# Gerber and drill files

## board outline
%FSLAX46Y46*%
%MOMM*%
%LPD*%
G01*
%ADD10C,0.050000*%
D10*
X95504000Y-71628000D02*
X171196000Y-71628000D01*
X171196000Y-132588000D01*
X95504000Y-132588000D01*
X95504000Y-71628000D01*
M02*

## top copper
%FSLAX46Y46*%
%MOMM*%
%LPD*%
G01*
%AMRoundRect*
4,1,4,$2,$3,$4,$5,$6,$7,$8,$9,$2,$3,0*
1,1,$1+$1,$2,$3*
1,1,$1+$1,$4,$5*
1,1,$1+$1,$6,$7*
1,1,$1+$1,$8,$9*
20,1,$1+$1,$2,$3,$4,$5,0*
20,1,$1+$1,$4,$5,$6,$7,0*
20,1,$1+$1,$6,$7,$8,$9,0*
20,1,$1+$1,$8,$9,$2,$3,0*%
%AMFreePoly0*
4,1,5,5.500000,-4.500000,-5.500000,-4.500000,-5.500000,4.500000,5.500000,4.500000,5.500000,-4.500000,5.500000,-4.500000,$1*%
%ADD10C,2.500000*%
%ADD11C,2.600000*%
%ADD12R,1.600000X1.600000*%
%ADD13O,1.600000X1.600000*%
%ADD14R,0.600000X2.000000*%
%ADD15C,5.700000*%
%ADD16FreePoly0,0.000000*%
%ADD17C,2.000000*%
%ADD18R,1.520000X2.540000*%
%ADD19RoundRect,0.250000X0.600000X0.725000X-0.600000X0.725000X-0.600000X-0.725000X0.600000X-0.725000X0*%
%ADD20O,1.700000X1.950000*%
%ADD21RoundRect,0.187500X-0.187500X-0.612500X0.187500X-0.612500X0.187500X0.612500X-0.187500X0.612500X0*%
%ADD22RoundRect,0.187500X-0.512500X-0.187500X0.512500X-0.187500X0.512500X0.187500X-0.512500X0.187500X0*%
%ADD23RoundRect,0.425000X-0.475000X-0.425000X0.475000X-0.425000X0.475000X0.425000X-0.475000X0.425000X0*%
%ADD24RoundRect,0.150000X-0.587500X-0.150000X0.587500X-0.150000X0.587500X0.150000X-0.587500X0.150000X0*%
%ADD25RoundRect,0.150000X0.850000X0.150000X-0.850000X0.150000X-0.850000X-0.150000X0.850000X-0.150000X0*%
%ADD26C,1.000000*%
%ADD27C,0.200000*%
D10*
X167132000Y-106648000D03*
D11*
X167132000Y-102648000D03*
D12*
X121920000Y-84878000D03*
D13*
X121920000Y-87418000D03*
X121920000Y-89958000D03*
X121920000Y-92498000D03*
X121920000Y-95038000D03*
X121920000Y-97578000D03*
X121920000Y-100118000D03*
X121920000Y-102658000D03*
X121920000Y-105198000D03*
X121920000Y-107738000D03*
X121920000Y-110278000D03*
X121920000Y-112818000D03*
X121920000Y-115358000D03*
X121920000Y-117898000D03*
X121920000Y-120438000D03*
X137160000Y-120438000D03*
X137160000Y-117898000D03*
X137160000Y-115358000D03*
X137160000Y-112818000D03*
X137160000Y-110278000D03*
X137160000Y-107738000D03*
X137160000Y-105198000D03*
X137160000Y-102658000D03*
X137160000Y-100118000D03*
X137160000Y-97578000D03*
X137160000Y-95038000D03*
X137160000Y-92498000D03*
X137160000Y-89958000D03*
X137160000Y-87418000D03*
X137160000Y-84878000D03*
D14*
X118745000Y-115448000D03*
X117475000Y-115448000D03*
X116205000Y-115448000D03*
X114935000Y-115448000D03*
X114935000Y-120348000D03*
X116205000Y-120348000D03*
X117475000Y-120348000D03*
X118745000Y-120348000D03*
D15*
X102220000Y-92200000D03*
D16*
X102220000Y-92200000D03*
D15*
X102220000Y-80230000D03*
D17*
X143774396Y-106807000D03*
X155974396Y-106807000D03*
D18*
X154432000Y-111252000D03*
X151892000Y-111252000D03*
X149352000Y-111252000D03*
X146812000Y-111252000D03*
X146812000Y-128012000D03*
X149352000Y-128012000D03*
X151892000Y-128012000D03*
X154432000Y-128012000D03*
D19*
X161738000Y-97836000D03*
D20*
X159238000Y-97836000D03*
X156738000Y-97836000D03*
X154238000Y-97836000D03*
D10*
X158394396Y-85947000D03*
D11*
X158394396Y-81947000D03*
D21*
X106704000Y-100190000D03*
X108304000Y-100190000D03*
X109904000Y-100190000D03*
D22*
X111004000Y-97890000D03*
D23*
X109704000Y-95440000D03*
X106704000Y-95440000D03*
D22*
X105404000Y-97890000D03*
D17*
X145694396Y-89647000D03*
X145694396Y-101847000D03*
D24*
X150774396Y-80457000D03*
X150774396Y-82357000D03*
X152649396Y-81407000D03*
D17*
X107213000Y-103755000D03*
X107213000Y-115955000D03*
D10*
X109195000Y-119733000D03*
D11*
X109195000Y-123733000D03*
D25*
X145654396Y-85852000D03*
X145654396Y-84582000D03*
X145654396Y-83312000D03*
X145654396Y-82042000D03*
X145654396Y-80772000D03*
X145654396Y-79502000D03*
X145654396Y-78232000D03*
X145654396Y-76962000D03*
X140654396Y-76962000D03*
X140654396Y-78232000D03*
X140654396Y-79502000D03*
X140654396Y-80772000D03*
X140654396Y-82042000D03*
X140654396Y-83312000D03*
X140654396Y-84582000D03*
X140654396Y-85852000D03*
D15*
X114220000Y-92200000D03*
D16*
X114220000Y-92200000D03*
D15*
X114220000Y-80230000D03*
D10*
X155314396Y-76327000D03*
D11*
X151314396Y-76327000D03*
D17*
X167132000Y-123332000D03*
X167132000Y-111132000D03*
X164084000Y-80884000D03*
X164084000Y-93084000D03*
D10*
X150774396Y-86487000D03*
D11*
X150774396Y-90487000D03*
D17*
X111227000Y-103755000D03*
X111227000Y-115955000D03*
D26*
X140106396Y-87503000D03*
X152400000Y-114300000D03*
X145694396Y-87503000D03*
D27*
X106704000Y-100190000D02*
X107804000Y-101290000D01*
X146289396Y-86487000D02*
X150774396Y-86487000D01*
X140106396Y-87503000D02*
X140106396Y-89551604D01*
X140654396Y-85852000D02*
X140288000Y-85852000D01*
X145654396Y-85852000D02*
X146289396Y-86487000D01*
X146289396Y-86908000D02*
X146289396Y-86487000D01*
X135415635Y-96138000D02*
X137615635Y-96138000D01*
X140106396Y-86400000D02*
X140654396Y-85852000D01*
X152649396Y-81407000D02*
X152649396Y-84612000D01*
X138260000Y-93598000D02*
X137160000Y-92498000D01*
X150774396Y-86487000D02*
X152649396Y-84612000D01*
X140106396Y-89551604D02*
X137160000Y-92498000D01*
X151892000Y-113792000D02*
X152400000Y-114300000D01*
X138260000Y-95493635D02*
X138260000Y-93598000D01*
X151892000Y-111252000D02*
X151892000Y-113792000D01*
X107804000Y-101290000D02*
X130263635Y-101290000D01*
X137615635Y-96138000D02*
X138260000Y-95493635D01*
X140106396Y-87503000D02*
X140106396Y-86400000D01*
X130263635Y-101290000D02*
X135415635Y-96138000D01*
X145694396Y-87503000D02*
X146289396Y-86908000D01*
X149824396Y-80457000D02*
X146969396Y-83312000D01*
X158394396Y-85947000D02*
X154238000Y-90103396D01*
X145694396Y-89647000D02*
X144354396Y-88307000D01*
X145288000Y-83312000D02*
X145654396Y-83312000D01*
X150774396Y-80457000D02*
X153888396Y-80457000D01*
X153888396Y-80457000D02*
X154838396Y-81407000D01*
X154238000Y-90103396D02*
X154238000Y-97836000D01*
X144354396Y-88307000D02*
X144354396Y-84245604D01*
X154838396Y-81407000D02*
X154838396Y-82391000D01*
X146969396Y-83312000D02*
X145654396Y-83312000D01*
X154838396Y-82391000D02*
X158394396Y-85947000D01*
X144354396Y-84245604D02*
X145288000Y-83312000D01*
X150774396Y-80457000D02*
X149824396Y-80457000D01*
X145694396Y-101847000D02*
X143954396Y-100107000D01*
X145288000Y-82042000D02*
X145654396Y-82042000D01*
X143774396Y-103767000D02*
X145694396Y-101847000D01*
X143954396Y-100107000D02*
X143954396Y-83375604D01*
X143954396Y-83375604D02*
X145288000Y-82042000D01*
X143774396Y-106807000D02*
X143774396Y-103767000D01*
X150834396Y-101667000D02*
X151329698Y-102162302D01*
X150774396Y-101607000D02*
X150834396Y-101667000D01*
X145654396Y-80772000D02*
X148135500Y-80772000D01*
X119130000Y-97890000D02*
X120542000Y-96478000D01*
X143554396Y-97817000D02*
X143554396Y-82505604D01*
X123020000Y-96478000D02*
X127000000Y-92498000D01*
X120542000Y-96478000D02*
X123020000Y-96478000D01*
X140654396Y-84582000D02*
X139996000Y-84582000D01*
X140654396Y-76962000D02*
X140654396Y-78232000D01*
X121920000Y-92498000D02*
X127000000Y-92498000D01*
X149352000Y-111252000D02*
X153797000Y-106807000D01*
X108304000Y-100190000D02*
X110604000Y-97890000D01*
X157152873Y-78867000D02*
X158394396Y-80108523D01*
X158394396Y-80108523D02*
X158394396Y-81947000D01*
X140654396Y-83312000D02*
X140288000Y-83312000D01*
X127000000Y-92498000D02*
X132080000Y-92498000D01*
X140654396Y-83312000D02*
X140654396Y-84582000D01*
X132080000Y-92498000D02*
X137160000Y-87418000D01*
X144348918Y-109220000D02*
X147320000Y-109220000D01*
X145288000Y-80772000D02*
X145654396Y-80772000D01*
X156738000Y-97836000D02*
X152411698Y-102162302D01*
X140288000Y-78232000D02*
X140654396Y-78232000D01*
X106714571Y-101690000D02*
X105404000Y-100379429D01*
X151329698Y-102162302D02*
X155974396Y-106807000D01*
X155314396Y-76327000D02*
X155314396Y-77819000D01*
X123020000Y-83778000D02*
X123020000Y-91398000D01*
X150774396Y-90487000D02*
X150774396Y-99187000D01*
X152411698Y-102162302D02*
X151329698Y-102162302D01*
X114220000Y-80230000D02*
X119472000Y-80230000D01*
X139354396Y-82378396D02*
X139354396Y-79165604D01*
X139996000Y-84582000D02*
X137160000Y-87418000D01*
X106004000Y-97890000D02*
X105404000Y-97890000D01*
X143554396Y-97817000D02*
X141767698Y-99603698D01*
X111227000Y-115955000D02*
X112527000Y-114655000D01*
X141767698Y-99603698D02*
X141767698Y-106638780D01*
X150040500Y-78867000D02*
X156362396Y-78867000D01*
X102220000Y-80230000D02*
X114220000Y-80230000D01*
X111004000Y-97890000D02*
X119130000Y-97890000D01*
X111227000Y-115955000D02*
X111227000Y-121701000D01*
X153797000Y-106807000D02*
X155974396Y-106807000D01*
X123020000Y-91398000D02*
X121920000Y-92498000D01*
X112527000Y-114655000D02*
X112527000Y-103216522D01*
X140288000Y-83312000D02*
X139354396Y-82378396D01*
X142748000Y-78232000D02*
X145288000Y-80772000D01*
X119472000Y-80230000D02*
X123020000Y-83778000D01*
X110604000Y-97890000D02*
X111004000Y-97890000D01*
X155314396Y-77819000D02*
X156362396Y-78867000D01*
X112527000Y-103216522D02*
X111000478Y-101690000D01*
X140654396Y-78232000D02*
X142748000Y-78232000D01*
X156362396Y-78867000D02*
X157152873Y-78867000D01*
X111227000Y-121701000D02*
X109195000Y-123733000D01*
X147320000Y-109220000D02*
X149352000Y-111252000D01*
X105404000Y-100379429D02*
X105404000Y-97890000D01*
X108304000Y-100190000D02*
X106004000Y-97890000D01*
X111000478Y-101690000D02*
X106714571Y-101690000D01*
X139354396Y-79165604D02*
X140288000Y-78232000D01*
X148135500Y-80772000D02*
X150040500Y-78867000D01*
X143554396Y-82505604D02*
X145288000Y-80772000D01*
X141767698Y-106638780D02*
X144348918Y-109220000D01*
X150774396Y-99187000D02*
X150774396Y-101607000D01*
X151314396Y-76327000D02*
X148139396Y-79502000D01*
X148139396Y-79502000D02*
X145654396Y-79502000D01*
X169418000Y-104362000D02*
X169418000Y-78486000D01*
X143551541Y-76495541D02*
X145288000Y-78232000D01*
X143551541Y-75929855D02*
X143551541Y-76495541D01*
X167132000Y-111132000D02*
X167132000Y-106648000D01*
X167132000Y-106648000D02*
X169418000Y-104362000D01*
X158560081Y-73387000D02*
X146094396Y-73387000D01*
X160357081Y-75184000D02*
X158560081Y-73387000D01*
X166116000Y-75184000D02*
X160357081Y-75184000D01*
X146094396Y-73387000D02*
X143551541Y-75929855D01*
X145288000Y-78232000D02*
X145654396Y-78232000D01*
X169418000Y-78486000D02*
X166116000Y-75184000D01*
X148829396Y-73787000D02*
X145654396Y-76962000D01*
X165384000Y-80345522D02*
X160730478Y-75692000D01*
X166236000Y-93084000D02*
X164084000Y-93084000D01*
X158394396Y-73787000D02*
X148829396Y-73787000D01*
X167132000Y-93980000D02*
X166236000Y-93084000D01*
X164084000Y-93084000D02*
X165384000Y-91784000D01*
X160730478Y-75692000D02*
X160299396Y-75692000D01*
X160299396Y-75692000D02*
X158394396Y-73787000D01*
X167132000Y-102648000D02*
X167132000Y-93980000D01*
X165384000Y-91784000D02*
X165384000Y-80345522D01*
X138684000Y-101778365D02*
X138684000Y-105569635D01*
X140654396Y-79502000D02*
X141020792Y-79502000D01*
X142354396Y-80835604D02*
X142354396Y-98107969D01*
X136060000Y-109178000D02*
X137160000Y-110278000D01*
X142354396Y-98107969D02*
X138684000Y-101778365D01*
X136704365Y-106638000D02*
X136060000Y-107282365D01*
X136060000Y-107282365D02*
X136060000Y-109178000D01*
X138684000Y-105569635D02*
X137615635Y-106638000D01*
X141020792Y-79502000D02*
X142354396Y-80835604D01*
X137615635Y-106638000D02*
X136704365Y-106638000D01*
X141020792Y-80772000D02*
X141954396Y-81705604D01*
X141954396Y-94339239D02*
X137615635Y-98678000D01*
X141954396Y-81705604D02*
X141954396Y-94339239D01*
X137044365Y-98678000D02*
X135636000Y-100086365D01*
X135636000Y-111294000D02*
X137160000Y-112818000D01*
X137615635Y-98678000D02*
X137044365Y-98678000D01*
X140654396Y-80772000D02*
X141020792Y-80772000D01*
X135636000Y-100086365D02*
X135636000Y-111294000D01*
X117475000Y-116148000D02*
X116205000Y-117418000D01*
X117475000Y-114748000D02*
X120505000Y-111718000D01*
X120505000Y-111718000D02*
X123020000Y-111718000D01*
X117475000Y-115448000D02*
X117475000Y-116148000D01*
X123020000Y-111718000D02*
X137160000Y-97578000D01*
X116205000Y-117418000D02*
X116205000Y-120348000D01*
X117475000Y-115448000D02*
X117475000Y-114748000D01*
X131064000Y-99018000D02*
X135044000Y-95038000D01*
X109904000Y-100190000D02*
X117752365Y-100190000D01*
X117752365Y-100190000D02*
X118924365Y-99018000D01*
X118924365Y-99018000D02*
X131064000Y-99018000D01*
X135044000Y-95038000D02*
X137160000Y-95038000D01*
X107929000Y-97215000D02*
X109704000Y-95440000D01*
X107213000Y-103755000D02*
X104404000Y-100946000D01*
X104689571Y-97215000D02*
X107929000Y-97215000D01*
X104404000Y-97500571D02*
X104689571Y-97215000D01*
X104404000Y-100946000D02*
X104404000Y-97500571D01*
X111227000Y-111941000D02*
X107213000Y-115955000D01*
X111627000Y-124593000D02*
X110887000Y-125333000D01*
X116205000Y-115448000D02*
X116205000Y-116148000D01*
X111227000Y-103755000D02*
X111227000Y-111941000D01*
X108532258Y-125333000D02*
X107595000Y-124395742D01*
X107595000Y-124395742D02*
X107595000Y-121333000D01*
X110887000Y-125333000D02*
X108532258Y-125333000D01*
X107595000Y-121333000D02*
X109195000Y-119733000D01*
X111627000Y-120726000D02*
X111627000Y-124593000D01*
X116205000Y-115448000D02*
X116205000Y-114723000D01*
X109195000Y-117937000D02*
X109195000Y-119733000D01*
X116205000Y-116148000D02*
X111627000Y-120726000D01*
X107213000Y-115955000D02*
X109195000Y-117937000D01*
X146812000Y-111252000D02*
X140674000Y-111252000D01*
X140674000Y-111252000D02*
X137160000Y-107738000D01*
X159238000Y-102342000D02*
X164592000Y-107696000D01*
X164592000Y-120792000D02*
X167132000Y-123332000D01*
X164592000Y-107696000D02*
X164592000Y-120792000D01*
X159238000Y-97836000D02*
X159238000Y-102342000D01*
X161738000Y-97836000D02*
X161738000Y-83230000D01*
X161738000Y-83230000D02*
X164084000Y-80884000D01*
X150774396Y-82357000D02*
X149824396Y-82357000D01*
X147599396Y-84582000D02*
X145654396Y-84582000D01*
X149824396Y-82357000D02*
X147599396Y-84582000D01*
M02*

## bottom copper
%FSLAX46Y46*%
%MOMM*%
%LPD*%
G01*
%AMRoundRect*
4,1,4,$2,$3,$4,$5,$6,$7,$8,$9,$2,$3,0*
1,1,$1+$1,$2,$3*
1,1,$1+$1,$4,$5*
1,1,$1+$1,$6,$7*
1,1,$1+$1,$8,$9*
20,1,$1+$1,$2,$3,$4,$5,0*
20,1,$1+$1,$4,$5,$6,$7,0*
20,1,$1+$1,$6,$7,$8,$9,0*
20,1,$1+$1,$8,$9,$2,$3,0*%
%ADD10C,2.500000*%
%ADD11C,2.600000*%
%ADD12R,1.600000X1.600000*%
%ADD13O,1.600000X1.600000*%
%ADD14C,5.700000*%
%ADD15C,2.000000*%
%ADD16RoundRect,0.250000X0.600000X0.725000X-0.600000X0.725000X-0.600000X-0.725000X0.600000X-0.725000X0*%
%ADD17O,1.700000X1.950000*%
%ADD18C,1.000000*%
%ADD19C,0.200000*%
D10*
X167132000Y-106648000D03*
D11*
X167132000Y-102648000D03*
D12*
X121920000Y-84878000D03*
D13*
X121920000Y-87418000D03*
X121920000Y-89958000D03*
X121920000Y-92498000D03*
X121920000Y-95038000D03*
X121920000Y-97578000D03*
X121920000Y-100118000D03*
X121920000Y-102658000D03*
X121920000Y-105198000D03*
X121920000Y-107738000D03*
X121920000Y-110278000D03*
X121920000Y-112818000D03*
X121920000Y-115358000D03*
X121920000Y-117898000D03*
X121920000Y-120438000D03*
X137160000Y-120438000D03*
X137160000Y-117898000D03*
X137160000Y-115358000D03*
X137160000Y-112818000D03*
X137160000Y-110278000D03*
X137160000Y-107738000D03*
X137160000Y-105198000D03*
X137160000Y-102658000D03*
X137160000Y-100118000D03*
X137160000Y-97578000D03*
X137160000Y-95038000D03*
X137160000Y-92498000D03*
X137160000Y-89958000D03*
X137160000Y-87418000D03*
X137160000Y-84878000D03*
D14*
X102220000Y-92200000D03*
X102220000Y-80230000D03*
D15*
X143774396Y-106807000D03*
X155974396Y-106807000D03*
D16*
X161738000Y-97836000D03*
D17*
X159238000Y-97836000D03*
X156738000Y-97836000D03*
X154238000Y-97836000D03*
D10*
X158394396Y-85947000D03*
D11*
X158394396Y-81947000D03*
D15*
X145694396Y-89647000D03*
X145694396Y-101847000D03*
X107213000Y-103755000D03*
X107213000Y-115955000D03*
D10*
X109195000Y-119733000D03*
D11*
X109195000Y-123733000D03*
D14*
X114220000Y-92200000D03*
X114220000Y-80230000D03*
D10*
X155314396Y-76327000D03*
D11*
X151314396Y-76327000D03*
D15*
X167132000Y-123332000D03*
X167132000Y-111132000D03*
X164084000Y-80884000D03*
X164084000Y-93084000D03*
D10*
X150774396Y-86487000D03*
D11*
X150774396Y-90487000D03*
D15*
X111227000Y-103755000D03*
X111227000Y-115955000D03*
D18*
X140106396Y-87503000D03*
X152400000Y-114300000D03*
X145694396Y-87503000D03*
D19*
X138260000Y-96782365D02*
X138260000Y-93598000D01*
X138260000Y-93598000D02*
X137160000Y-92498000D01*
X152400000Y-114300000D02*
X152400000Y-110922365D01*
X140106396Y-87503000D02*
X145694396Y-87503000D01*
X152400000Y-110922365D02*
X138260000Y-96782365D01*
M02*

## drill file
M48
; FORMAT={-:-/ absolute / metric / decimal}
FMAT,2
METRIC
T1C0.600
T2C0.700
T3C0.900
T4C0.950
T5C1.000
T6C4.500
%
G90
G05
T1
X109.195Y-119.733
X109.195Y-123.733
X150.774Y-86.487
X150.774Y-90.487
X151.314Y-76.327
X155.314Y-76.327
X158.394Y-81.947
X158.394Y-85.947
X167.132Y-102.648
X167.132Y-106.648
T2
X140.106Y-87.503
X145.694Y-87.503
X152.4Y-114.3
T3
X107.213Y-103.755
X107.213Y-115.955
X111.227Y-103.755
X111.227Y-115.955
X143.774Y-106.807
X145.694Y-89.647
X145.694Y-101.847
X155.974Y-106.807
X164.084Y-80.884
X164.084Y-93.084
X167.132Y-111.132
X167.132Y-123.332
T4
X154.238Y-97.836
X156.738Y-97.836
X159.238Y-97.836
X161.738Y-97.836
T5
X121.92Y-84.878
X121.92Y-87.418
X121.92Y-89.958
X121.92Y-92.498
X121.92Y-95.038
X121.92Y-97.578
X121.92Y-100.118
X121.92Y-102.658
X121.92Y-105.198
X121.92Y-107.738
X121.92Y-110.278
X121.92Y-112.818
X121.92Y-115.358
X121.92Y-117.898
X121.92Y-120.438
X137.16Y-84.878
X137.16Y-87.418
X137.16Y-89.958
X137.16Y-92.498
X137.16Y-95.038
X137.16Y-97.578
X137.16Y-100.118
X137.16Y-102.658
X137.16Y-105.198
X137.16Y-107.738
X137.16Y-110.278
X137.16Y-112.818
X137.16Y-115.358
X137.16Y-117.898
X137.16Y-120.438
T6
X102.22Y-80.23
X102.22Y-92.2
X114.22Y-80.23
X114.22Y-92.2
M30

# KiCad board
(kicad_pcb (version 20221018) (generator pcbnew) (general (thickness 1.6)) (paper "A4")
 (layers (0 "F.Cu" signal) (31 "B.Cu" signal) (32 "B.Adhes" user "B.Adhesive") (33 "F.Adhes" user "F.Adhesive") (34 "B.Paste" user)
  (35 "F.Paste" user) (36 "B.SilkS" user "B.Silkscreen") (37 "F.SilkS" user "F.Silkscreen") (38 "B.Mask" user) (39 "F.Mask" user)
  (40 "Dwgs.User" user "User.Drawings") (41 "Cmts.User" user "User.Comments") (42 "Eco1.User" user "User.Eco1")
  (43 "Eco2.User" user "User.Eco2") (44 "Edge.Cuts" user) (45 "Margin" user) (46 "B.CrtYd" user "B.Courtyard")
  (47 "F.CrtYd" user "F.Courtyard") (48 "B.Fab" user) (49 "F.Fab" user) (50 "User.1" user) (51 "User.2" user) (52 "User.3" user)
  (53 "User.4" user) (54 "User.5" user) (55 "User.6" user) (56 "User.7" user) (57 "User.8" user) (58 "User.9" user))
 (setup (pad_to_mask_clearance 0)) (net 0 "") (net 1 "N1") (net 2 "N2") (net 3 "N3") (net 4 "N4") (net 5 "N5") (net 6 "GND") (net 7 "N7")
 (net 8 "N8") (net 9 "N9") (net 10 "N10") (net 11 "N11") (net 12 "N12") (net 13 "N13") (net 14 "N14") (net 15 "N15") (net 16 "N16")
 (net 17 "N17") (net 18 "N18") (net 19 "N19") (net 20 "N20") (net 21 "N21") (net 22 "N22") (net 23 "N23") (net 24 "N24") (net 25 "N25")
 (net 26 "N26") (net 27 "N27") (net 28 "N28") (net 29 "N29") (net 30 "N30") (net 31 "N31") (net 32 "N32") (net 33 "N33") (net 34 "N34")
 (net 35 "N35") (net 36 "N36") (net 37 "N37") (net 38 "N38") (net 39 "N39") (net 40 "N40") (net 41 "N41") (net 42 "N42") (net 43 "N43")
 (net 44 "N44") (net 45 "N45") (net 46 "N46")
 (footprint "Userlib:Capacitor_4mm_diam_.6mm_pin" (layer "F.Cu") (at 167.132 104.648 90)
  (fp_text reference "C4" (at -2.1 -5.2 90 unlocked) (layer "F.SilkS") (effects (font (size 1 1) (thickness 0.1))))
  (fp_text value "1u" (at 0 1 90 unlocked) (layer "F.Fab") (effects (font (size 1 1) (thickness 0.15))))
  (pad "1" thru_hole circle (at -2 0 90) (size 2.5 2.5) (drill 0.6) (layers "*.Cu" "*.Mask") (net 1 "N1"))
  (pad "2" thru_hole circle (at 2 0 90) (size 2.6 2.6) (drill 0.6) (layers "*.Cu" "*.Mask") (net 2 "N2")))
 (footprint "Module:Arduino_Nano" (layer "F.Cu") (at 121.92 84.878)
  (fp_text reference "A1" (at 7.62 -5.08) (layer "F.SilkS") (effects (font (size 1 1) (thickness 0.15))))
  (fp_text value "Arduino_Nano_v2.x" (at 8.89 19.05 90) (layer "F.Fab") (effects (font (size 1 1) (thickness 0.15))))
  (pad "1" thru_hole rect (at 0 0) (size 1.6 1.6) (drill 1) (layers "*.Cu" "*.Mask") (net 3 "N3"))
  (pad "2" thru_hole oval (at 0 2.54) (size 1.6 1.6) (drill 1) (layers "*.Cu" "*.Mask") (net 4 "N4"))
  (pad "3" thru_hole oval (at 0 5.08) (size 1.6 1.6) (drill 1) (layers "*.Cu" "*.Mask") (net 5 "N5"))
  (pad "4" thru_hole oval (at 0 7.62) (size 1.6 1.6) (drill 1) (layers "*.Cu" "*.Mask") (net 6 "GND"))
  (pad "5" thru_hole oval (at 0 10.16) (size 1.6 1.6) (drill 1) (layers "*.Cu" "*.Mask") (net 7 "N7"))
  (pad "6" thru_hole oval (at 0 12.7) (size 1.6 1.6) (drill 1) (layers "*.Cu" "*.Mask") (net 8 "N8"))
  (pad "7" thru_hole oval (at 0 15.24) (size 1.6 1.6) (drill 1) (layers "*.Cu" "*.Mask") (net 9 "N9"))
  (pad "8" thru_hole oval (at 0 17.78) (size 1.6 1.6) (drill 1) (layers "*.Cu" "*.Mask") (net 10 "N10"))
  (pad "9" thru_hole oval (at 0 20.32) (size 1.6 1.6) (drill 1) (layers "*.Cu" "*.Mask") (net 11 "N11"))
  (pad "10" thru_hole oval (at 0 22.86) (size 1.6 1.6) (drill 1) (layers "*.Cu" "*.Mask") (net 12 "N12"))
  (pad "11" thru_hole oval (at 0 25.4) (size 1.6 1.6) (drill 1) (layers "*.Cu" "*.Mask") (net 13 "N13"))
  (pad "12" thru_hole oval (at 0 27.94) (size 1.6 1.6) (drill 1) (layers "*.Cu" "*.Mask") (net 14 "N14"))
  (pad "13" thru_hole oval (at 0 30.48) (size 1.6 1.6) (drill 1) (layers "*.Cu" "*.Mask") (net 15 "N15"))
  (pad "14" thru_hole oval (at 0 33.02) (size 1.6 1.6) (drill 1) (layers "*.Cu" "*.Mask") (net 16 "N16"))
  (pad "15" thru_hole oval (at 0 35.56) (size 1.6 1.6) (drill 1) (layers "*.Cu" "*.Mask") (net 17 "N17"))
  (pad "16" thru_hole oval (at 15.24 35.56) (size 1.6 1.6) (drill 1) (layers "*.Cu" "*.Mask") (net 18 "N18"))
  (pad "17" thru_hole oval (at 15.24 33.02) (size 1.6 1.6) (drill 1) (layers "*.Cu" "*.Mask") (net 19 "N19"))
  (pad "18" thru_hole oval (at 15.24 30.48) (size 1.6 1.6) (drill 1) (layers "*.Cu" "*.Mask") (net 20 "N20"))
  (pad "19" thru_hole oval (at 15.24 27.94) (size 1.6 1.6) (drill 1) (layers "*.Cu" "*.Mask") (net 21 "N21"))
  (pad "20" thru_hole oval (at 15.24 25.4) (size 1.6 1.6) (drill 1) (layers "*.Cu" "*.Mask") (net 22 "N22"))
  (pad "21" thru_hole oval (at 15.24 22.86) (size 1.6 1.6) (drill 1) (layers "*.Cu" "*.Mask") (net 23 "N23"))
  (pad "22" thru_hole oval (at 15.24 20.32) (size 1.6 1.6) (drill 1) (layers "*.Cu" "*.Mask") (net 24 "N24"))
  (pad "23" thru_hole oval (at 15.24 17.78) (size 1.6 1.6) (drill 1) (layers "*.Cu" "*.Mask") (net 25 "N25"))
  (pad "24" thru_hole oval (at 15.24 15.24) (size 1.6 1.6) (drill 1) (layers "*.Cu" "*.Mask") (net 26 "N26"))
  (pad "25" thru_hole oval (at 15.24 12.7) (size 1.6 1.6) (drill 1) (layers "*.Cu" "*.Mask") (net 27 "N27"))
  (pad "26" thru_hole oval (at 15.24 10.16) (size 1.6 1.6) (drill 1) (layers "*.Cu" "*.Mask") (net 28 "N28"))
  (pad "27" thru_hole oval (at 15.24 7.62) (size 1.6 1.6) (drill 1) (layers "*.Cu" "*.Mask") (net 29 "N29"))
  (pad "28" thru_hole oval (at 15.24 5.08) (size 1.6 1.6) (drill 1) (layers "*.Cu" "*.Mask") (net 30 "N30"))
  (pad "29" thru_hole oval (at 15.24 2.54) (size 1.6 1.6) (drill 1) (layers "*.Cu" "*.Mask") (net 6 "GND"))
  (pad "30" thru_hole oval (at 15.24 0) (size 1.6 1.6) (drill 1) (layers "*.Cu" "*.Mask") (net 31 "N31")))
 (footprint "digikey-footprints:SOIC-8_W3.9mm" (layer "F.Cu") (at 116.84 117.898 180)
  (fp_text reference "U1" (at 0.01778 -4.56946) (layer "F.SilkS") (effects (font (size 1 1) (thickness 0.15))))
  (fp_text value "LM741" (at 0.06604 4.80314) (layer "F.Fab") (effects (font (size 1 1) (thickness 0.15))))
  (pad "1" smd rect (at -1.905 2.45 180) (size 0.6 2) (layers "F.Cu" "F.Paste" "F.Mask") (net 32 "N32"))
  (pad "2" smd rect (at -0.635 2.45 180) (size 0.6 2) (layers "F.Cu" "F.Paste" "F.Mask") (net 27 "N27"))
  (pad "3" smd rect (at 0.635 2.45 180) (size 0.6 2) (layers "F.Cu" "F.Paste" "F.Mask") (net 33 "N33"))
  (pad "4" smd rect (at 1.905 2.45 180) (size 0.6 2) (layers "F.Cu" "F.Paste" "F.Mask") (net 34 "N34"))
  (pad "5" smd rect (at 1.905 -2.45 180) (size 0.6 2) (layers "F.Cu" "F.Paste" "F.Mask") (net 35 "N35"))
  (pad "6" smd rect (at 0.635 -2.45 180) (size 0.6 2) (layers "F.Cu" "F.Paste" "F.Mask") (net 27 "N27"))
  (pad "7" smd rect (at -0.635 -2.45 180) (size 0.6 2) (layers "F.Cu" "F.Paste" "F.Mask") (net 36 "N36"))
  (pad "8" smd rect (at -1.905 -2.45 180) (size 0.6 2) (layers "F.Cu" "F.Paste" "F.Mask") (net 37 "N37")))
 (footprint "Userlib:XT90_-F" (layer "F.Cu") (at 102.3 96.52)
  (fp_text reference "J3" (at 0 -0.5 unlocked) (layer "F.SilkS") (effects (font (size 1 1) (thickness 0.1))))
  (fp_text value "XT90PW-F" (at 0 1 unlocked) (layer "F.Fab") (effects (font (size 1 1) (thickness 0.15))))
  (pad "1" thru_hole circle (at -0.08 -4.32) (size 5.7 5.7) (drill 4.5) (layers "*.Cu" "*.Mask") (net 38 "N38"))
  (pad "1" smd custom (at -0.08 -4.32) (size 11 9) (layers "F.Cu" "F.Paste" "F.Mask") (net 38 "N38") (thermal_bridge_angle 45)
   (options (clearance outline) (anchor rect)) (primitives))
  (pad "2" thru_hole circle (at -0.08 -16.29) (size 5.7 5.7) (drill 4.5) (layers "*.Cu" "*.Mask") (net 6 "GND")))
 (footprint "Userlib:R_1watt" (layer "F.Cu") (at 150.774396 106.807 180)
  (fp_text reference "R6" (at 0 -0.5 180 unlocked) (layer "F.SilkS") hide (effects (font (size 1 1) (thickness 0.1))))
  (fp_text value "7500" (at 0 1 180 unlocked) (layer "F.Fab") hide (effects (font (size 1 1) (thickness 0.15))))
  (pad "1" thru_hole circle (at 7 0 180) (size 2 2) (drill 0.9) (layers "*.Cu" "*.Mask") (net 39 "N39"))
  (pad "2" thru_hole circle (at -5.2 0 180) (size 2 2) (drill 0.9) (layers "*.Cu" "*.Mask") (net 6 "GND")))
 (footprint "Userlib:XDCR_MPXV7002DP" (layer "F.Cu") (at 150.622 119.632 -90)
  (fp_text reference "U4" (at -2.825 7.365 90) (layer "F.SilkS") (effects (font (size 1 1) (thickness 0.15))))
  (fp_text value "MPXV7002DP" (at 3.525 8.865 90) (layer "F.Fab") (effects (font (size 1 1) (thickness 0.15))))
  (pad "1" smd rect (at -8.38 -3.81 270) (size 2.54 1.52) (layers "F.Cu" "F.Paste" "F.Mask") (solder_mask_margin 0.102))
  (pad "2" smd rect (at -8.38 -1.27 270) (size 2.54 1.52) (layers "F.Cu" "F.Paste" "F.Mask") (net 29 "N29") (solder_mask_margin 0.102))
  (pad "3" smd rect (at -8.38 1.27 270) (size 2.54 1.52) (layers "F.Cu" "F.Paste" "F.Mask") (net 6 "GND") (solder_mask_margin 0.102))
  (pad "4" smd rect (at -8.38 3.81 270) (size 2.54 1.52) (layers "F.Cu" "F.Paste" "F.Mask") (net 23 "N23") (solder_mask_margin 0.102))
  (pad "5" smd rect (at 8.38 3.81 270) (size 2.54 1.52) (layers "F.Cu" "F.Paste" "F.Mask") (solder_mask_margin 0.102))
  (pad "6" smd rect (at 8.38 1.27 270) (size 2.54 1.52) (layers "F.Cu" "F.Paste" "F.Mask") (solder_mask_margin 0.102))
  (pad "7" smd rect (at 8.38 -1.27 270) (size 2.54 1.52) (layers "F.Cu" "F.Paste" "F.Mask") (solder_mask_margin 0.102))
  (pad "8" smd rect (at 8.38 -3.81 270) (size 2.54 1.52) (layers "F.Cu" "F.Paste" "F.Mask") (solder_mask_margin 0.102)))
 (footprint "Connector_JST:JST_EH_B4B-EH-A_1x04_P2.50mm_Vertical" (layer "F.Cu") (at 161.738 97.836 180)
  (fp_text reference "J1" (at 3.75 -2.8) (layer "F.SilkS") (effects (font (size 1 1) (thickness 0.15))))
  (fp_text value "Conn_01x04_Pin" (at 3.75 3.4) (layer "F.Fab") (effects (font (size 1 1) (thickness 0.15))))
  (pad "1" thru_hole roundrect (at 0 0 180) (size 1.7 1.95) (drill 0.95) (layers "*.Cu" "*.Mask") (roundrect_rratio 0.147059) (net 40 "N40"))
  (pad "2" thru_hole oval (at 2.5 0 180) (size 1.7 1.95) (drill 0.95) (layers "*.Cu" "*.Mask") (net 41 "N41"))
  (pad "3" thru_hole oval (at 5 0 180) (size 1.7 1.95) (drill 0.95) (layers "*.Cu" "*.Mask") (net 6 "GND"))
  (pad "4" thru_hole oval (at 7.5 0 180) (size 1.7 1.95) (drill 0.95) (layers "*.Cu" "*.Mask") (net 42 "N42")))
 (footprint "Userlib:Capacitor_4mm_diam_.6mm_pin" (layer "F.Cu") (at 158.394396 83.947 90)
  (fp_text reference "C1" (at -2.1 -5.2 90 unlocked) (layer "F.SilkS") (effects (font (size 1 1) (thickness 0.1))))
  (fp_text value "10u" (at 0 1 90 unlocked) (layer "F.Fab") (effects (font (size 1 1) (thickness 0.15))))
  (pad "1" thru_hole circle (at -2 0 90) (size 2.5 2.5) (drill 0.6) (layers "*.Cu" "*.Mask") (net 42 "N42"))
  (pad "2" thru_hole circle (at 2 0 90) (size 2.6 2.6) (drill 0.6) (layers "*.Cu" "*.Mask") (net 6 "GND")))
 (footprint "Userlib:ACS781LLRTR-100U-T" (layer "F.Cu") (at 105.004 100.09)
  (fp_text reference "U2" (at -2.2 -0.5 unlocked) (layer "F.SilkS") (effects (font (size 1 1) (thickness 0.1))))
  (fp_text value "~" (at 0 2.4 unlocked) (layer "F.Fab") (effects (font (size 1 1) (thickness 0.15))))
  (pad "1" smd roundrect (at 1.7 0.1) (size 0.75 1.6) (layers "F.Cu" "F.Paste" "F.Mask") (roundrect_rratio 0.25) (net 29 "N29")
   (thermal_bridge_angle 45))
  (pad "2" smd roundrect (at 3.3 0.1) (size 0.75 1.6) (layers "F.Cu" "F.Paste" "F.Mask") (roundrect_rratio 0.25) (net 6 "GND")
   (thermal_bridge_angle 45))
  (pad "3" smd roundrect (at 4.9 0.1) (size 0.75 1.6) (layers "F.Cu" "F.Paste" "F.Mask") (roundrect_rratio 0.25) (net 28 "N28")
   (thermal_bridge_angle 45))
  (pad "4" smd roundrect (at 6 -2.2) (size 1.4 0.75) (layers "F.Cu" "F.Paste" "F.Mask") (roundrect_rratio 0.25) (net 6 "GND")
   (thermal_bridge_angle 45))
  (pad "5" smd roundrect (at 4.7 -4.65) (size 1.8 1.7) (layers "F.Cu" "F.Paste" "F.Mask") (roundrect_rratio 0.25) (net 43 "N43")
   (thermal_bridge_angle 45))
  (pad "6" smd roundrect (at 1.7 -4.65) (size 1.8 1.7) (layers "F.Cu" "F.Paste" "F.Mask") (roundrect_rratio 0.25) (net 38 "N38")
   (thermal_bridge_angle 45))
  (pad "7" smd roundrect (at 0.4 -2.2) (size 1.4 0.75) (layers "F.Cu" "F.Paste" "F.Mask") (roundrect_rratio 0.25) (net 6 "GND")
   (thermal_bridge_angle 45)))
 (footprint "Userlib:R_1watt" (layer "F.Cu") (at 145.694396 96.647 90)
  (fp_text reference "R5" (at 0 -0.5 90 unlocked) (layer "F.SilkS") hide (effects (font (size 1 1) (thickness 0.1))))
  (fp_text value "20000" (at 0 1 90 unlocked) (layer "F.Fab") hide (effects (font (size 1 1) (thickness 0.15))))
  (pad "1" thru_hole circle (at 7 0 90) (size 2 2) (drill 0.9) (layers "*.Cu" "*.Mask") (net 42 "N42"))
  (pad "2" thru_hole circle (at -5.2 0 90) (size 2 2) (drill 0.9) (layers "*.Cu" "*.Mask") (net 39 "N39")))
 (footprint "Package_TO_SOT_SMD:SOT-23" (layer "F.Cu") (at 151.711896 81.407)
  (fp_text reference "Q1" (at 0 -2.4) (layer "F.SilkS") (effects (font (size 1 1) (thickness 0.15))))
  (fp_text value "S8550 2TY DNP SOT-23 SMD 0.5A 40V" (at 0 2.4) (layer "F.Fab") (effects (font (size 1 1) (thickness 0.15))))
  (pad "1" smd roundrect (at -0.9375 -0.95) (size 1.475 0.6) (layers "F.Cu" "F.Paste" "F.Mask") (roundrect_rratio 0.25) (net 42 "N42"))
  (pad "2" smd roundrect (at -0.9375 0.95) (size 1.475 0.6) (layers "F.Cu" "F.Paste" "F.Mask") (roundrect_rratio 0.25) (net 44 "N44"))
  (pad "3" smd roundrect (at 0.9375 0) (size 1.475 0.6) (layers "F.Cu" "F.Paste" "F.Mask") (roundrect_rratio 0.25) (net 29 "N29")))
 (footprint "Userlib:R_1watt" (layer "F.Cu") (at 107.213 110.755 90)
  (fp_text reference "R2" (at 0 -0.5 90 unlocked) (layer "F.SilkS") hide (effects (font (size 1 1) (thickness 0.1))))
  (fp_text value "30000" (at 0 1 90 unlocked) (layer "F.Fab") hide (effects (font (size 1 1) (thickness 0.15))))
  (pad "1" thru_hole circle (at 7 0 90) (size 2 2) (drill 0.9) (layers "*.Cu" "*.Mask") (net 43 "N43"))
  (pad "2" thru_hole circle (at -5.2 0 90) (size 2 2) (drill 0.9) (layers "*.Cu" "*.Mask") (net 33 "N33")))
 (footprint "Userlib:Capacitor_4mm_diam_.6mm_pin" (layer "F.Cu") (at 109.195 121.733 -90)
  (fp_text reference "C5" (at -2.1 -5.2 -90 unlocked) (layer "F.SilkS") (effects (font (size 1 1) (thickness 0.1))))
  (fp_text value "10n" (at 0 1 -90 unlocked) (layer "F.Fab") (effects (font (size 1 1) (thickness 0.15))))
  (pad "1" thru_hole circle (at -2 0 270) (size 2.5 2.5) (drill 0.6) (layers "*.Cu" "*.Mask") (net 33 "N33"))
  (pad "2" thru_hole circle (at 2 0 270) (size 2.6 2.6) (drill 0.6) (layers "*.Cu" "*.Mask") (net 6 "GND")))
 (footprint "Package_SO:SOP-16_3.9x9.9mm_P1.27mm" (layer "F.Cu") (at 143.154396 81.407 180)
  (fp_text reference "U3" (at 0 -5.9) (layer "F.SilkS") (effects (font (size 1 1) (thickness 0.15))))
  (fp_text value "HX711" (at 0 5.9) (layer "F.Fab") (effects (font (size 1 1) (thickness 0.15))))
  (pad "1" smd roundrect (at -2.5 -4.445 180) (size 2 0.6) (layers "F.Cu" "F.Paste" "F.Mask") (roundrect_rratio 0.25) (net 29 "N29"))
  (pad "2" smd roundrect (at -2.5 -3.175 180) (size 2 0.6) (layers "F.Cu" "F.Paste" "F.Mask") (roundrect_rratio 0.25) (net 44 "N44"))
  (pad "3" smd roundrect (at -2.5 -1.905 180) (size 2 0.6) (layers "F.Cu" "F.Paste" "F.Mask") (roundrect_rratio 0.25) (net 42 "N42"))
  (pad "4" smd roundrect (at -2.5 -0.635 180) (size 2 0.6) (layers "F.Cu" "F.Paste" "F.Mask") (roundrect_rratio 0.25) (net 39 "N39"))
  (pad "5" smd roundrect (at -2.5 0.635 180) (size 2 0.6) (layers "F.Cu" "F.Paste" "F.Mask") (roundrect_rratio 0.25) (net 6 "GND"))
  (pad "6" smd roundrect (at -2.5 1.905 180) (size 2 0.6) (layers "F.Cu" "F.Paste" "F.Mask") (roundrect_rratio 0.25) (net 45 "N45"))
  (pad "7" smd roundrect (at -2.5 3.175 180) (size 2 0.6) (layers "F.Cu" "F.Paste" "F.Mask") (roundrect_rratio 0.25) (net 1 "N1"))
  (pad "8" smd roundrect (at -2.5 4.445 180) (size 2 0.6) (layers "F.Cu" "F.Paste" "F.Mask") (roundrect_rratio 0.25) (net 2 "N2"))
  (pad "9" smd roundrect (at 2.5 4.445 180) (size 2 0.6) (layers "F.Cu" "F.Paste" "F.Mask") (roundrect_rratio 0.25) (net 6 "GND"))
  (pad "10" smd roundrect (at 2.5 3.175 180) (size 2 0.6) (layers "F.Cu" "F.Paste" "F.Mask") (roundrect_rratio 0.25) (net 6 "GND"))
  (pad "11" smd roundrect (at 2.5 1.905 180) (size 2 0.6) (layers "F.Cu" "F.Paste" "F.Mask") (roundrect_rratio 0.25) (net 22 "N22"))
  (pad "12" smd roundrect (at 2.5 0.635 180) (size 2 0.6) (layers "F.Cu" "F.Paste" "F.Mask") (roundrect_rratio 0.25) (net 21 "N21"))
  (pad "13" smd roundrect (at 2.5 -0.635 180) (size 2 0.6) (layers "F.Cu" "F.Paste" "F.Mask") (roundrect_rratio 0.25) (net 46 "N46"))
  (pad "14" smd roundrect (at 2.5 -1.905 180) (size 2 0.6) (layers "F.Cu" "F.Paste" "F.Mask") (roundrect_rratio 0.25) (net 6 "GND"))
  (pad "15" smd roundrect (at 2.5 -3.175 180) (size 2 0.6) (layers "F.Cu" "F.Paste" "F.Mask") (roundrect_rratio 0.25) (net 6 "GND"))
  (pad "16" smd roundrect (at 2.5 -4.445 180) (size 2 0.6) (layers "F.Cu" "F.Paste" "F.Mask") (roundrect_rratio 0.25) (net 29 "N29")))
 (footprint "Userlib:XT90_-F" (layer "F.Cu") (at 114.3 96.52)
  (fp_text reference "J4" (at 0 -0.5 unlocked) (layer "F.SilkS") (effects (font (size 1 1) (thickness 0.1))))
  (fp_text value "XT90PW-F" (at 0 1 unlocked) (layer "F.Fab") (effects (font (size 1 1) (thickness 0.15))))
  (pad "1" thru_hole circle (at -0.08 -4.32) (size 5.7 5.7) (drill 4.5) (layers "*.Cu" "*.Mask") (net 43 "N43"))
  (pad "1" smd custom (at -0.08 -4.32) (size 11 9) (layers "F.Cu" "F.Paste" "F.Mask") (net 43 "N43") (thermal_bridge_angle 45)
   (options (clearance outline) (anchor rect)) (primitives))
  (pad "2" thru_hole circle (at -0.08 -16.29) (size 5.7 5.7) (drill 4.5) (layers "*.Cu" "*.Mask") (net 6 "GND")))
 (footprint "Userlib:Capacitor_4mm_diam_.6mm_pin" (layer "F.Cu") (at 153.314396 76.327 180)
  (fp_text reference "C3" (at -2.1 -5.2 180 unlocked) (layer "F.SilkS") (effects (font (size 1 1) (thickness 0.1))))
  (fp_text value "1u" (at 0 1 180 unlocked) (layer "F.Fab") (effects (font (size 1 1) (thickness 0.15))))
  (pad "1" thru_hole circle (at -2 0 180) (size 2.5 2.5) (drill 0.6) (layers "*.Cu" "*.Mask") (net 6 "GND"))
  (pad "2" thru_hole circle (at 2 0 180) (size 2.6 2.6) (drill 0.6) (layers "*.Cu" "*.Mask") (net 45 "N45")))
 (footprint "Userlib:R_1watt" (layer "F.Cu") (at 167.132 116.332 -90)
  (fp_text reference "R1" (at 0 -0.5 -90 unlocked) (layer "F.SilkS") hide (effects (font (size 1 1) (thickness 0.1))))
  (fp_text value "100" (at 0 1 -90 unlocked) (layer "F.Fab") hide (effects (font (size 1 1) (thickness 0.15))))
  (pad "1" thru_hole circle (at 7 0 270) (size 2 2) (drill 0.9) (layers "*.Cu" "*.Mask") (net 41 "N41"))
  (pad "2" thru_hole circle (at -5.2 0 270) (size 2 2) (drill 0.9) (layers "*.Cu" "*.Mask") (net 1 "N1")))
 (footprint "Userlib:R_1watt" (layer "F.Cu") (at 164.084 87.884 90)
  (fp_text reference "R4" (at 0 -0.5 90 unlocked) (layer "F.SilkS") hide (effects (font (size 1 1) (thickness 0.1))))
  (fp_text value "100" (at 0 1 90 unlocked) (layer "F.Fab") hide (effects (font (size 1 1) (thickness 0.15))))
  (pad "1" thru_hole circle (at 7 0 90) (size 2 2) (drill 0.9) (layers "*.Cu" "*.Mask") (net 40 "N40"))
  (pad "2" thru_hole circle (at -5.2 0 90) (size 2 2) (drill 0.9) (layers "*.Cu" "*.Mask") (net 2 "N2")))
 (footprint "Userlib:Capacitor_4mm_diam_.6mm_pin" (layer "F.Cu") (at 150.774396 88.487 -90)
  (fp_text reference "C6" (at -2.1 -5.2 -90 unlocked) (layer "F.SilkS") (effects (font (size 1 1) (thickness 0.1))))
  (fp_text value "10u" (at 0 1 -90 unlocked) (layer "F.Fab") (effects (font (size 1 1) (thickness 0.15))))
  (pad "1" thru_hole circle (at -2 0 270) (size 2.5 2.5) (drill 0.6) (layers "*.Cu" "*.Mask") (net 29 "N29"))
  (pad "2" thru_hole circle (at 2 0 270) (size 2.6 2.6) (drill 0.6) (layers "*.Cu" "*.Mask") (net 6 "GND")))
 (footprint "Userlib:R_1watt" (layer "F.Cu") (at 111.227 110.755 90)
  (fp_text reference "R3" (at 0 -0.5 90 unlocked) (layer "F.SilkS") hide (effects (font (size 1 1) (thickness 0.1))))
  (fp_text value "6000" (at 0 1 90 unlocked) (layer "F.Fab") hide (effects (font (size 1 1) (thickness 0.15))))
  (pad "1" thru_hole circle (at 7 0 90) (size 2 2) (drill 0.9) (layers "*.Cu" "*.Mask") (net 33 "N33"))
  (pad "2" thru_hole circle (at -5.2 0 90) (size 2 2) (drill 0.9) (layers "*.Cu" "*.Mask") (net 6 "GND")))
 (gr_rect (start 95.504 71.628) (end 171.196 132.588) (stroke (width 0.05) (type default)) (fill none) (layer "Edge.Cuts"))
 (segment (start 106.704 100.19) (end 107.804 101.29) (width 0.2) (layer "F.Cu") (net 29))
 (segment (start 146.289396 86.487) (end 150.774396 86.487) (width 0.2) (layer "F.Cu") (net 29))
 (segment (start 140.106396 87.503) (end 140.106396 89.551604) (width 0.2) (layer "F.Cu") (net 29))
 (segment (start 140.654396 85.852) (end 140.288 85.852) (width 0.2) (layer "F.Cu") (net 29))
 (segment (start 145.654396 85.852) (end 146.289396 86.487) (width 0.2) (layer "F.Cu") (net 29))
 (segment (start 146.289396 86.908) (end 146.289396 86.487) (width 0.2) (layer "F.Cu") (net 29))
 (segment (start 135.415635 96.138) (end 137.615635 96.138) (width 0.2) (layer "F.Cu") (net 29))
 (segment (start 140.106396 86.4) (end 140.654396 85.852) (width 0.2) (layer "F.Cu") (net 29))
 (segment (start 152.649396 81.407) (end 152.649396 84.612) (width 0.2) (layer "F.Cu") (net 29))
 (segment (start 138.26 93.598) (end 137.16 92.498) (width 0.2) (layer "F.Cu") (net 29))
 (segment (start 150.774396 86.487) (end 152.649396 84.612) (width 0.2) (layer "F.Cu") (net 29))
 (segment (start 140.106396 89.551604) (end 137.16 92.498) (width 0.2) (layer "F.Cu") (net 29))
 (segment (start 151.892 113.792) (end 152.4 114.3) (width 0.2) (layer "F.Cu") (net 29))
 (segment (start 138.26 95.493635) (end 138.26 93.598) (width 0.2) (layer "F.Cu") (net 29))
 (segment (start 151.892 111.252) (end 151.892 113.792) (width 0.2) (layer "F.Cu") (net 29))
 (segment (start 107.804 101.29) (end 130.263635 101.29) (width 0.2) (layer "F.Cu") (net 29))
 (segment (start 137.615635 96.138) (end 138.26 95.493635) (width 0.2) (layer "F.Cu") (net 29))
 (segment (start 140.106396 87.503) (end 140.106396 86.4) (width 0.2) (layer "F.Cu") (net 29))
 (segment (start 130.263635 101.29) (end 135.415635 96.138) (width 0.2) (layer "F.Cu") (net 29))
 (segment (start 145.694396 87.503) (end 146.289396 86.908) (width 0.2) (layer "F.Cu") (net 29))
 (via (at 140.106396 87.503) (size 1) (drill 0.7) (layers "F.Cu" "B.Cu") (free) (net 29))
 (via (at 152.4 114.3) (size 1) (drill 0.7) (layers "F.Cu" "B.Cu") (free) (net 29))
 (via (at 145.694396 87.503) (size 1) (drill 0.7) (layers "F.Cu" "B.Cu") (free) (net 29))
 (segment (start 138.26 96.782365) (end 138.26 93.598) (width 0.2) (layer "B.Cu") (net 29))
 (segment (start 138.26 93.598) (end 137.16 92.498) (width 0.2) (layer "B.Cu") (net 29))
 (segment (start 152.4 114.3) (end 152.4 110.922365) (width 0.2) (layer "B.Cu") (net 29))
 (segment (start 140.106396 87.503) (end 145.694396 87.503) (width 0.2) (layer "B.Cu") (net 29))
 (segment (start 152.4 110.922365) (end 138.26 96.782365) (width 0.2) (layer "B.Cu") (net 29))
 (segment (start 149.824396 80.457) (end 146.969396 83.312) (width 0.2) (layer "F.Cu") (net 42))
 (segment (start 158.394396 85.947) (end 154.238 90.103396) (width 0.2) (layer "F.Cu") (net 42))
 (segment (start 145.694396 89.647) (end 144.354396 88.307) (width 0.2) (layer "F.Cu") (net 42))
 (segment (start 145.288 83.312) (end 145.654396 83.312) (width 0.2) (layer "F.Cu") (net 42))
 (segment (start 150.774396 80.457) (end 153.888396 80.457) (width 0.2) (layer "F.Cu") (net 42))
 (segment (start 153.888396 80.457) (end 154.838396 81.407) (width 0.2) (layer "F.Cu") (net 42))
 (segment (start 154.238 90.103396) (end 154.238 97.836) (width 0.2) (layer "F.Cu") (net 42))
 (segment (start 144.354396 88.307) (end 144.354396 84.245604) (width 0.2) (layer "F.Cu") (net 42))
 (segment (start 154.838396 81.407) (end 154.838396 82.391) (width 0.2) (layer "F.Cu") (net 42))
 (segment (start 146.969396 83.312) (end 145.654396 83.312) (width 0.2) (layer "F.Cu") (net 42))
 (segment (start 154.838396 82.391) (end 158.394396 85.947) (width 0.2) (layer "F.Cu") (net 42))
 (segment (start 144.354396 84.245604) (end 145.288 83.312) (width 0.2) (layer "F.Cu") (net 42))
 (segment (start 150.774396 80.457) (end 149.824396 80.457) (width 0.2) (layer "F.Cu") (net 42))
 (segment (start 145.694396 101.847) (end 143.954396 100.107) (width 0.2) (layer "F.Cu") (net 39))
 (segment (start 145.288 82.042) (end 145.654396 82.042) (width 0.2) (layer "F.Cu") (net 39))
 (segment (start 143.774396 103.767) (end 145.694396 101.847) (width 0.2) (layer "F.Cu") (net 39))
 (segment (start 143.954396 100.107) (end 143.954396 83.375604) (width 0.2) (layer "F.Cu") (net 39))
 (segment (start 143.954396 83.375604) (end 145.288 82.042) (width 0.2) (layer "F.Cu") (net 39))
 (segment (start 143.774396 106.807) (end 143.774396 103.767) (width 0.2) (layer "F.Cu") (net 39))
 (segment (start 150.834396 101.667) (end 151.329698 102.162302) (width 0.2) (layer "F.Cu") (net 6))
 (segment (start 150.774396 101.607) (end 150.834396 101.667) (width 0.2) (layer "F.Cu") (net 6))
 (segment (start 145.654396 80.772) (end 148.1355 80.772) (width 0.2) (layer "F.Cu") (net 6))
 (segment (start 119.13 97.89) (end 120.542 96.478) (width 0.2) (layer "F.Cu") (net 6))
 (segment (start 143.554396 97.817) (end 143.554396 82.505604) (width 0.2) (layer "F.Cu") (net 6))
 (segment (start 123.02 96.478) (end 127 92.498) (width 0.2) (layer "F.Cu") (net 6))
 (segment (start 120.542 96.478) (end 123.02 96.478) (width 0.2) (layer "F.Cu") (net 6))
 (segment (start 140.654396 84.582) (end 139.996 84.582) (width 0.2) (layer "F.Cu") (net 6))
 (segment (start 140.654396 76.962) (end 140.654396 78.232) (width 0.2) (layer "F.Cu") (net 6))
 (segment (start 121.92 92.498) (end 127 92.498) (width 0.2) (layer "F.Cu") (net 6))
 (segment (start 149.352 111.252) (end 153.797 106.807) (width 0.2) (layer "F.Cu") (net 6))
 (segment (start 108.304 100.19) (end 110.604 97.89) (width 0.2) (layer "F.Cu") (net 6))
 (segment (start 157.152873 78.867) (end 158.394396 80.108523) (width 0.2) (layer "F.Cu") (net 6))
 (segment (start 158.394396 80.108523) (end 158.394396 81.947) (width 0.2) (layer "F.Cu") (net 6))
 (segment (start 140.654396 83.312) (end 140.288 83.312) (width 0.2) (layer "F.Cu") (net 6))
 (segment (start 127 92.498) (end 132.08 92.498) (width 0.2) (layer "F.Cu") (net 6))
 (segment (start 140.654396 83.312) (end 140.654396 84.582) (width 0.2) (layer "F.Cu") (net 6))
 (segment (start 132.08 92.498) (end 137.16 87.418) (width 0.2) (layer "F.Cu") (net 6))
 (segment (start 144.348918 109.22) (end 147.32 109.22) (width 0.2) (layer "F.Cu") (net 6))
 (segment (start 145.288 80.772) (end 145.654396 80.772) (width 0.2) (layer "F.Cu") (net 6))
 (segment (start 156.738 97.836) (end 152.411698 102.162302) (width 0.2) (layer "F.Cu") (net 6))
 (segment (start 140.288 78.232) (end 140.654396 78.232) (width 0.2) (layer "F.Cu") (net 6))
 (segment (start 106.714571 101.69) (end 105.404 100.379429) (width 0.2) (layer "F.Cu") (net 6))
 (segment (start 151.329698 102.162302) (end 155.974396 106.807) (width 0.2) (layer "F.Cu") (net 6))
 (segment (start 155.314396 76.327) (end 155.314396 77.819) (width 0.2) (layer "F.Cu") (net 6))
 (segment (start 123.02 83.778) (end 123.02 91.398) (width 0.2) (layer "F.Cu") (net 6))
 (segment (start 150.774396 90.487) (end 150.774396 99.187) (width 0.2) (layer "F.Cu") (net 6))
 (segment (start 152.411698 102.162302) (end 151.329698 102.162302) (width 0.2) (layer "F.Cu") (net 6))
 (segment (start 114.22 80.23) (end 119.472 80.23) (width 0.2) (layer "F.Cu") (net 6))
 (segment (start 139.354396 82.378396) (end 139.354396 79.165604) (width 0.2) (layer "F.Cu") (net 6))
 (segment (start 139.996 84.582) (end 137.16 87.418) (width 0.2) (layer "F.Cu") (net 6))
 (segment (start 106.004 97.89) (end 105.404 97.89) (width 0.2) (layer "F.Cu") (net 6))
 (segment (start 143.554396 97.817) (end 141.767698 99.603698) (width 0.2) (layer "F.Cu") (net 6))
 (segment (start 111.227 115.955) (end 112.527 114.655) (width 0.2) (layer "F.Cu") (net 6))
 (segment (start 141.767698 99.603698) (end 141.767698 106.63878) (width 0.2) (layer "F.Cu") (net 6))
 (segment (start 150.0405 78.867) (end 156.362396 78.867) (width 0.2) (layer "F.Cu") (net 6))
 (segment (start 102.22 80.23) (end 114.22 80.23) (width 0.2) (layer "F.Cu") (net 6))
 (segment (start 111.004 97.89) (end 119.13 97.89) (width 0.2) (layer "F.Cu") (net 6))
 (segment (start 111.227 115.955) (end 111.227 121.701) (width 0.2) (layer "F.Cu") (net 6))
 (segment (start 153.797 106.807) (end 155.974396 106.807) (width 0.2) (layer "F.Cu") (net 6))
 (segment (start 123.02 91.398) (end 121.92 92.498) (width 0.2) (layer "F.Cu") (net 6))
 (segment (start 112.527 114.655) (end 112.527 103.216522) (width 0.2) (layer "F.Cu") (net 6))
 (segment (start 140.288 83.312) (end 139.354396 82.378396) (width 0.2) (layer "F.Cu") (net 6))
 (segment (start 142.748 78.232) (end 145.288 80.772) (width 0.2) (layer "F.Cu") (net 6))
 (segment (start 119.472 80.23) (end 123.02 83.778) (width 0.2) (layer "F.Cu") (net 6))
 (segment (start 110.604 97.89) (end 111.004 97.89) (width 0.2) (layer "F.Cu") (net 6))
 (segment (start 155.314396 77.819) (end 156.362396 78.867) (width 0.2) (layer "F.Cu") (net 6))
 (segment (start 112.527 103.216522) (end 111.000478 101.69) (width 0.2) (layer "F.Cu") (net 6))
 (segment (start 140.654396 78.232) (end 142.748 78.232) (width 0.2) (layer "F.Cu") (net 6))
 (segment (start 156.362396 78.867) (end 157.152873 78.867) (width 0.2) (layer "F.Cu") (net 6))
 (segment (start 111.227 121.701) (end 109.195 123.733) (width 0.2) (layer "F.Cu") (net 6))
 (segment (start 147.32 109.22) (end 149.352 111.252) (width 0.2) (layer "F.Cu") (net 6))
 (segment (start 105.404 100.379429) (end 105.404 97.89) (width 0.2) (layer "F.Cu") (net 6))
 (segment (start 108.304 100.19) (end 106.004 97.89) (width 0.2) (layer "F.Cu") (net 6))
 (segment (start 111.000478 101.69) (end 106.714571 101.69) (width 0.2) (layer "F.Cu") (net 6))
 (segment (start 139.354396 79.165604) (end 140.288 78.232) (width 0.2) (layer "F.Cu") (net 6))
 (segment (start 148.1355 80.772) (end 150.0405 78.867) (width 0.2) (layer "F.Cu") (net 6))
 (segment (start 143.554396 82.505604) (end 145.288 80.772) (width 0.2) (layer "F.Cu") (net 6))
 (segment (start 141.767698 106.63878) (end 144.348918 109.22) (width 0.2) (layer "F.Cu") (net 6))
 (segment (start 150.774396 99.187) (end 150.774396 101.607) (width 0.2) (layer "F.Cu") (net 6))
 (segment (start 151.314396 76.327) (end 148.139396 79.502) (width 0.2) (layer "F.Cu") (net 45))
 (segment (start 148.139396 79.502) (end 145.654396 79.502) (width 0.2) (layer "F.Cu") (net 45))
 (segment (start 169.418 104.362) (end 169.418 78.486) (width 0.2) (layer "F.Cu") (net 1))
 (segment (start 143.551541 76.495541) (end 145.288 78.232) (width 0.2) (layer "F.Cu") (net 1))
 (segment (start 143.551541 75.929855) (end 143.551541 76.495541) (width 0.2) (layer "F.Cu") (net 1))
 (segment (start 167.132 111.132) (end 167.132 106.648) (width 0.2) (layer "F.Cu") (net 1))
 (segment (start 167.132 106.648) (end 169.418 104.362) (width 0.2) (layer "F.Cu") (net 1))
 (segment (start 158.560081 73.387) (end 146.094396 73.387) (width 0.2) (layer "F.Cu") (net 1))
 (segment (start 160.357081 75.184) (end 158.560081 73.387) (width 0.2) (layer "F.Cu") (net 1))
 (segment (start 166.116 75.184) (end 160.357081 75.184) (width 0.2) (layer "F.Cu") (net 1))
 (segment (start 146.094396 73.387) (end 143.551541 75.929855) (width 0.2) (layer "F.Cu") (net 1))
 (segment (start 145.288 78.232) (end 145.654396 78.232) (width 0.2) (layer "F.Cu") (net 1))
 (segment (start 169.418 78.486) (end 166.116 75.184) (width 0.2) (layer "F.Cu") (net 1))
 (segment (start 148.829396 73.787) (end 145.654396 76.962) (width 0.2) (layer "F.Cu") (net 2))
 (segment (start 165.384 80.345522) (end 160.730478 75.692) (width 0.2) (layer "F.Cu") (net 2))
 (segment (start 166.236 93.084) (end 164.084 93.084) (width 0.2) (layer "F.Cu") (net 2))
 (segment (start 158.394396 73.787) (end 148.829396 73.787) (width 0.2) (layer "F.Cu") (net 2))
 (segment (start 167.132 93.98) (end 166.236 93.084) (width 0.2) (layer "F.Cu") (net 2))
 (segment (start 164.084 93.084) (end 165.384 91.784) (width 0.2) (layer "F.Cu") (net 2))
 (segment (start 160.730478 75.692) (end 160.299396 75.692) (width 0.2) (layer "F.Cu") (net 2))
 (segment (start 160.299396 75.692) (end 158.394396 73.787) (width 0.2) (layer "F.Cu") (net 2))
 (segment (start 167.132 102.648) (end 167.132 93.98) (width 0.2) (layer "F.Cu") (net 2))
 (segment (start 165.384 91.784) (end 165.384 80.345522) (width 0.2) (layer "F.Cu") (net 2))
 (segment (start 138.684 101.778365) (end 138.684 105.569635) (width 0.2) (layer "F.Cu") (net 22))
 (segment (start 140.654396 79.502) (end 141.020792 79.502) (width 0.2) (layer "F.Cu") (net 22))
 (segment (start 142.354396 80.835604) (end 142.354396 98.107969) (width 0.2) (layer "F.Cu") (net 22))
 (segment (start 136.06 109.178) (end 137.16 110.278) (width 0.2) (layer "F.Cu") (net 22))
 (segment (start 142.354396 98.107969) (end 138.684 101.778365) (width 0.2) (layer "F.Cu") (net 22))
 (segment (start 136.704365 106.638) (end 136.06 107.282365) (width 0.2) (layer "F.Cu") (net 22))
 (segment (start 136.06 107.282365) (end 136.06 109.178) (width 0.2) (layer "F.Cu") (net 22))
 (segment (start 138.684 105.569635) (end 137.615635 106.638) (width 0.2) (layer "F.Cu") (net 22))
 (segment (start 141.020792 79.502) (end 142.354396 80.835604) (width 0.2) (layer "F.Cu") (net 22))
 (segment (start 137.615635 106.638) (end 136.704365 106.638) (width 0.2) (layer "F.Cu") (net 22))
 (segment (start 141.020792 80.772) (end 141.954396 81.705604) (width 0.2) (layer "F.Cu") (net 21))
 (segment (start 141.954396 94.339239) (end 137.615635 98.678) (width 0.2) (layer "F.Cu") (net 21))
 (segment (start 141.954396 81.705604) (end 141.954396 94.339239) (width 0.2) (layer "F.Cu") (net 21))
 (segment (start 137.044365 98.678) (end 135.636 100.086365) (width 0.2) (layer "F.Cu") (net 21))
 (segment (start 135.636 111.294) (end 137.16 112.818) (width 0.2) (layer "F.Cu") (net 21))
 (segment (start 137.615635 98.678) (end 137.044365 98.678) (width 0.2) (layer "F.Cu") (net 21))
 (segment (start 140.654396 80.772) (end 141.020792 80.772) (width 0.2) (layer "F.Cu") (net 21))
 (segment (start 135.636 100.086365) (end 135.636 111.294) (width 0.2) (layer "F.Cu") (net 21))
 (segment (start 117.475 116.148) (end 116.205 117.418) (width 0.2) (layer "F.Cu") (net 27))
 (segment (start 117.475 114.748) (end 120.505 111.718) (width 0.2) (layer "F.Cu") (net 27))
 (segment (start 120.505 111.718) (end 123.02 111.718) (width 0.2) (layer "F.Cu") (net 27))
 (segment (start 117.475 115.448) (end 117.475 116.148) (width 0.2) (layer "F.Cu") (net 27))
 (segment (start 123.02 111.718) (end 137.16 97.578) (width 0.2) (layer "F.Cu") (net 27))
 (segment (start 116.205 117.418) (end 116.205 120.348) (width 0.2) (layer "F.Cu") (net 27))
 (segment (start 117.475 115.448) (end 117.475 114.748) (width 0.2) (layer "F.Cu") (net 27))
 (segment (start 131.064 99.018) (end 135.044 95.038) (width 0.2) (layer "F.Cu") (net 28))
 (segment (start 109.904 100.19) (end 117.752365 100.19) (width 0.2) (layer "F.Cu") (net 28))
 (segment (start 117.752365 100.19) (end 118.924365 99.018) (width 0.2) (layer "F.Cu") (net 28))
 (segment (start 118.924365 99.018) (end 131.064 99.018) (width 0.2) (layer "F.Cu") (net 28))
 (segment (start 135.044 95.038) (end 137.16 95.038) (width 0.2) (layer "F.Cu") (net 28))
 (segment (start 107.929 97.215) (end 109.704 95.44) (width 0.2) (layer "F.Cu") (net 43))
 (segment (start 107.213 103.755) (end 104.404 100.946) (width 0.2) (layer "F.Cu") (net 43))
 (segment (start 104.689571 97.215) (end 107.929 97.215) (width 0.2) (layer "F.Cu") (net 43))
 (segment (start 104.404 97.500571) (end 104.689571 97.215) (width 0.2) (layer "F.Cu") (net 43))
 (segment (start 104.404 100.946) (end 104.404 97.500571) (width 0.2) (layer "F.Cu") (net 43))
 (segment (start 111.227 111.941) (end 107.213 115.955) (width 0.2) (layer "F.Cu") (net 33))
 (segment (start 111.627 124.593) (end 110.887 125.333) (width 0.2) (layer "F.Cu") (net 33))
 (segment (start 116.205 115.448) (end 116.205 116.148) (width 0.2) (layer "F.Cu") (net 33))
 (segment (start 111.227 103.755) (end 111.227 111.941) (width 0.2) (layer "F.Cu") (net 33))
 (segment (start 108.532258 125.333) (end 107.595 124.395742) (width 0.2) (layer "F.Cu") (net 33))
 (segment (start 107.595 124.395742) (end 107.595 121.333) (width 0.2) (layer "F.Cu") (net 33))
 (segment (start 110.887 125.333) (end 108.532258 125.333) (width 0.2) (layer "F.Cu") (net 33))
 (segment (start 107.595 121.333) (end 109.195 119.733) (width 0.2) (layer "F.Cu") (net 33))
 (segment (start 111.627 120.726) (end 111.627 124.593) (width 0.2) (layer "F.Cu") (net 33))
 (segment (start 116.205 115.448) (end 116.205 114.723) (width 0.2) (layer "F.Cu") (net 33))
 (segment (start 109.195 117.937) (end 109.195 119.733) (width 0.2) (layer "F.Cu") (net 33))
 (segment (start 116.205 116.148) (end 111.627 120.726) (width 0.2) (layer "F.Cu") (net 33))
 (segment (start 107.213 115.955) (end 109.195 117.937) (width 0.2) (layer "F.Cu") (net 33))
 (segment (start 146.812 111.252) (end 140.674 111.252) (width 0.2) (layer "F.Cu") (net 23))
 (segment (start 140.674 111.252) (end 137.16 107.738) (width 0.2) (layer "F.Cu") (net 23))
 (segment (start 159.238 102.342) (end 164.592 107.696) (width 0.2) (layer "F.Cu") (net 41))
 (segment (start 164.592 120.792) (end 167.132 123.332) (width 0.2) (layer "F.Cu") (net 41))
 (segment (start 164.592 107.696) (end 164.592 120.792) (width 0.2) (layer "F.Cu") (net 41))
 (segment (start 159.238 97.836) (end 159.238 102.342) (width 0.2) (layer "F.Cu") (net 41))
 (segment (start 161.738 97.836) (end 161.738 83.23) (width 0.2) (layer "F.Cu") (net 40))
 (segment (start 161.738 83.23) (end 164.084 80.884) (width 0.2) (layer "F.Cu") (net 40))
 (segment (start 150.774396 82.357) (end 149.824396 82.357) (width 0.2) (layer "F.Cu") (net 44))
 (segment (start 147.599396 84.582) (end 145.654396 84.582) (width 0.2) (layer "F.Cu") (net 44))
 (segment (start 149.824396 82.357) (end 147.599396 84.582) (width 0.2) (layer "F.Cu") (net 44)))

